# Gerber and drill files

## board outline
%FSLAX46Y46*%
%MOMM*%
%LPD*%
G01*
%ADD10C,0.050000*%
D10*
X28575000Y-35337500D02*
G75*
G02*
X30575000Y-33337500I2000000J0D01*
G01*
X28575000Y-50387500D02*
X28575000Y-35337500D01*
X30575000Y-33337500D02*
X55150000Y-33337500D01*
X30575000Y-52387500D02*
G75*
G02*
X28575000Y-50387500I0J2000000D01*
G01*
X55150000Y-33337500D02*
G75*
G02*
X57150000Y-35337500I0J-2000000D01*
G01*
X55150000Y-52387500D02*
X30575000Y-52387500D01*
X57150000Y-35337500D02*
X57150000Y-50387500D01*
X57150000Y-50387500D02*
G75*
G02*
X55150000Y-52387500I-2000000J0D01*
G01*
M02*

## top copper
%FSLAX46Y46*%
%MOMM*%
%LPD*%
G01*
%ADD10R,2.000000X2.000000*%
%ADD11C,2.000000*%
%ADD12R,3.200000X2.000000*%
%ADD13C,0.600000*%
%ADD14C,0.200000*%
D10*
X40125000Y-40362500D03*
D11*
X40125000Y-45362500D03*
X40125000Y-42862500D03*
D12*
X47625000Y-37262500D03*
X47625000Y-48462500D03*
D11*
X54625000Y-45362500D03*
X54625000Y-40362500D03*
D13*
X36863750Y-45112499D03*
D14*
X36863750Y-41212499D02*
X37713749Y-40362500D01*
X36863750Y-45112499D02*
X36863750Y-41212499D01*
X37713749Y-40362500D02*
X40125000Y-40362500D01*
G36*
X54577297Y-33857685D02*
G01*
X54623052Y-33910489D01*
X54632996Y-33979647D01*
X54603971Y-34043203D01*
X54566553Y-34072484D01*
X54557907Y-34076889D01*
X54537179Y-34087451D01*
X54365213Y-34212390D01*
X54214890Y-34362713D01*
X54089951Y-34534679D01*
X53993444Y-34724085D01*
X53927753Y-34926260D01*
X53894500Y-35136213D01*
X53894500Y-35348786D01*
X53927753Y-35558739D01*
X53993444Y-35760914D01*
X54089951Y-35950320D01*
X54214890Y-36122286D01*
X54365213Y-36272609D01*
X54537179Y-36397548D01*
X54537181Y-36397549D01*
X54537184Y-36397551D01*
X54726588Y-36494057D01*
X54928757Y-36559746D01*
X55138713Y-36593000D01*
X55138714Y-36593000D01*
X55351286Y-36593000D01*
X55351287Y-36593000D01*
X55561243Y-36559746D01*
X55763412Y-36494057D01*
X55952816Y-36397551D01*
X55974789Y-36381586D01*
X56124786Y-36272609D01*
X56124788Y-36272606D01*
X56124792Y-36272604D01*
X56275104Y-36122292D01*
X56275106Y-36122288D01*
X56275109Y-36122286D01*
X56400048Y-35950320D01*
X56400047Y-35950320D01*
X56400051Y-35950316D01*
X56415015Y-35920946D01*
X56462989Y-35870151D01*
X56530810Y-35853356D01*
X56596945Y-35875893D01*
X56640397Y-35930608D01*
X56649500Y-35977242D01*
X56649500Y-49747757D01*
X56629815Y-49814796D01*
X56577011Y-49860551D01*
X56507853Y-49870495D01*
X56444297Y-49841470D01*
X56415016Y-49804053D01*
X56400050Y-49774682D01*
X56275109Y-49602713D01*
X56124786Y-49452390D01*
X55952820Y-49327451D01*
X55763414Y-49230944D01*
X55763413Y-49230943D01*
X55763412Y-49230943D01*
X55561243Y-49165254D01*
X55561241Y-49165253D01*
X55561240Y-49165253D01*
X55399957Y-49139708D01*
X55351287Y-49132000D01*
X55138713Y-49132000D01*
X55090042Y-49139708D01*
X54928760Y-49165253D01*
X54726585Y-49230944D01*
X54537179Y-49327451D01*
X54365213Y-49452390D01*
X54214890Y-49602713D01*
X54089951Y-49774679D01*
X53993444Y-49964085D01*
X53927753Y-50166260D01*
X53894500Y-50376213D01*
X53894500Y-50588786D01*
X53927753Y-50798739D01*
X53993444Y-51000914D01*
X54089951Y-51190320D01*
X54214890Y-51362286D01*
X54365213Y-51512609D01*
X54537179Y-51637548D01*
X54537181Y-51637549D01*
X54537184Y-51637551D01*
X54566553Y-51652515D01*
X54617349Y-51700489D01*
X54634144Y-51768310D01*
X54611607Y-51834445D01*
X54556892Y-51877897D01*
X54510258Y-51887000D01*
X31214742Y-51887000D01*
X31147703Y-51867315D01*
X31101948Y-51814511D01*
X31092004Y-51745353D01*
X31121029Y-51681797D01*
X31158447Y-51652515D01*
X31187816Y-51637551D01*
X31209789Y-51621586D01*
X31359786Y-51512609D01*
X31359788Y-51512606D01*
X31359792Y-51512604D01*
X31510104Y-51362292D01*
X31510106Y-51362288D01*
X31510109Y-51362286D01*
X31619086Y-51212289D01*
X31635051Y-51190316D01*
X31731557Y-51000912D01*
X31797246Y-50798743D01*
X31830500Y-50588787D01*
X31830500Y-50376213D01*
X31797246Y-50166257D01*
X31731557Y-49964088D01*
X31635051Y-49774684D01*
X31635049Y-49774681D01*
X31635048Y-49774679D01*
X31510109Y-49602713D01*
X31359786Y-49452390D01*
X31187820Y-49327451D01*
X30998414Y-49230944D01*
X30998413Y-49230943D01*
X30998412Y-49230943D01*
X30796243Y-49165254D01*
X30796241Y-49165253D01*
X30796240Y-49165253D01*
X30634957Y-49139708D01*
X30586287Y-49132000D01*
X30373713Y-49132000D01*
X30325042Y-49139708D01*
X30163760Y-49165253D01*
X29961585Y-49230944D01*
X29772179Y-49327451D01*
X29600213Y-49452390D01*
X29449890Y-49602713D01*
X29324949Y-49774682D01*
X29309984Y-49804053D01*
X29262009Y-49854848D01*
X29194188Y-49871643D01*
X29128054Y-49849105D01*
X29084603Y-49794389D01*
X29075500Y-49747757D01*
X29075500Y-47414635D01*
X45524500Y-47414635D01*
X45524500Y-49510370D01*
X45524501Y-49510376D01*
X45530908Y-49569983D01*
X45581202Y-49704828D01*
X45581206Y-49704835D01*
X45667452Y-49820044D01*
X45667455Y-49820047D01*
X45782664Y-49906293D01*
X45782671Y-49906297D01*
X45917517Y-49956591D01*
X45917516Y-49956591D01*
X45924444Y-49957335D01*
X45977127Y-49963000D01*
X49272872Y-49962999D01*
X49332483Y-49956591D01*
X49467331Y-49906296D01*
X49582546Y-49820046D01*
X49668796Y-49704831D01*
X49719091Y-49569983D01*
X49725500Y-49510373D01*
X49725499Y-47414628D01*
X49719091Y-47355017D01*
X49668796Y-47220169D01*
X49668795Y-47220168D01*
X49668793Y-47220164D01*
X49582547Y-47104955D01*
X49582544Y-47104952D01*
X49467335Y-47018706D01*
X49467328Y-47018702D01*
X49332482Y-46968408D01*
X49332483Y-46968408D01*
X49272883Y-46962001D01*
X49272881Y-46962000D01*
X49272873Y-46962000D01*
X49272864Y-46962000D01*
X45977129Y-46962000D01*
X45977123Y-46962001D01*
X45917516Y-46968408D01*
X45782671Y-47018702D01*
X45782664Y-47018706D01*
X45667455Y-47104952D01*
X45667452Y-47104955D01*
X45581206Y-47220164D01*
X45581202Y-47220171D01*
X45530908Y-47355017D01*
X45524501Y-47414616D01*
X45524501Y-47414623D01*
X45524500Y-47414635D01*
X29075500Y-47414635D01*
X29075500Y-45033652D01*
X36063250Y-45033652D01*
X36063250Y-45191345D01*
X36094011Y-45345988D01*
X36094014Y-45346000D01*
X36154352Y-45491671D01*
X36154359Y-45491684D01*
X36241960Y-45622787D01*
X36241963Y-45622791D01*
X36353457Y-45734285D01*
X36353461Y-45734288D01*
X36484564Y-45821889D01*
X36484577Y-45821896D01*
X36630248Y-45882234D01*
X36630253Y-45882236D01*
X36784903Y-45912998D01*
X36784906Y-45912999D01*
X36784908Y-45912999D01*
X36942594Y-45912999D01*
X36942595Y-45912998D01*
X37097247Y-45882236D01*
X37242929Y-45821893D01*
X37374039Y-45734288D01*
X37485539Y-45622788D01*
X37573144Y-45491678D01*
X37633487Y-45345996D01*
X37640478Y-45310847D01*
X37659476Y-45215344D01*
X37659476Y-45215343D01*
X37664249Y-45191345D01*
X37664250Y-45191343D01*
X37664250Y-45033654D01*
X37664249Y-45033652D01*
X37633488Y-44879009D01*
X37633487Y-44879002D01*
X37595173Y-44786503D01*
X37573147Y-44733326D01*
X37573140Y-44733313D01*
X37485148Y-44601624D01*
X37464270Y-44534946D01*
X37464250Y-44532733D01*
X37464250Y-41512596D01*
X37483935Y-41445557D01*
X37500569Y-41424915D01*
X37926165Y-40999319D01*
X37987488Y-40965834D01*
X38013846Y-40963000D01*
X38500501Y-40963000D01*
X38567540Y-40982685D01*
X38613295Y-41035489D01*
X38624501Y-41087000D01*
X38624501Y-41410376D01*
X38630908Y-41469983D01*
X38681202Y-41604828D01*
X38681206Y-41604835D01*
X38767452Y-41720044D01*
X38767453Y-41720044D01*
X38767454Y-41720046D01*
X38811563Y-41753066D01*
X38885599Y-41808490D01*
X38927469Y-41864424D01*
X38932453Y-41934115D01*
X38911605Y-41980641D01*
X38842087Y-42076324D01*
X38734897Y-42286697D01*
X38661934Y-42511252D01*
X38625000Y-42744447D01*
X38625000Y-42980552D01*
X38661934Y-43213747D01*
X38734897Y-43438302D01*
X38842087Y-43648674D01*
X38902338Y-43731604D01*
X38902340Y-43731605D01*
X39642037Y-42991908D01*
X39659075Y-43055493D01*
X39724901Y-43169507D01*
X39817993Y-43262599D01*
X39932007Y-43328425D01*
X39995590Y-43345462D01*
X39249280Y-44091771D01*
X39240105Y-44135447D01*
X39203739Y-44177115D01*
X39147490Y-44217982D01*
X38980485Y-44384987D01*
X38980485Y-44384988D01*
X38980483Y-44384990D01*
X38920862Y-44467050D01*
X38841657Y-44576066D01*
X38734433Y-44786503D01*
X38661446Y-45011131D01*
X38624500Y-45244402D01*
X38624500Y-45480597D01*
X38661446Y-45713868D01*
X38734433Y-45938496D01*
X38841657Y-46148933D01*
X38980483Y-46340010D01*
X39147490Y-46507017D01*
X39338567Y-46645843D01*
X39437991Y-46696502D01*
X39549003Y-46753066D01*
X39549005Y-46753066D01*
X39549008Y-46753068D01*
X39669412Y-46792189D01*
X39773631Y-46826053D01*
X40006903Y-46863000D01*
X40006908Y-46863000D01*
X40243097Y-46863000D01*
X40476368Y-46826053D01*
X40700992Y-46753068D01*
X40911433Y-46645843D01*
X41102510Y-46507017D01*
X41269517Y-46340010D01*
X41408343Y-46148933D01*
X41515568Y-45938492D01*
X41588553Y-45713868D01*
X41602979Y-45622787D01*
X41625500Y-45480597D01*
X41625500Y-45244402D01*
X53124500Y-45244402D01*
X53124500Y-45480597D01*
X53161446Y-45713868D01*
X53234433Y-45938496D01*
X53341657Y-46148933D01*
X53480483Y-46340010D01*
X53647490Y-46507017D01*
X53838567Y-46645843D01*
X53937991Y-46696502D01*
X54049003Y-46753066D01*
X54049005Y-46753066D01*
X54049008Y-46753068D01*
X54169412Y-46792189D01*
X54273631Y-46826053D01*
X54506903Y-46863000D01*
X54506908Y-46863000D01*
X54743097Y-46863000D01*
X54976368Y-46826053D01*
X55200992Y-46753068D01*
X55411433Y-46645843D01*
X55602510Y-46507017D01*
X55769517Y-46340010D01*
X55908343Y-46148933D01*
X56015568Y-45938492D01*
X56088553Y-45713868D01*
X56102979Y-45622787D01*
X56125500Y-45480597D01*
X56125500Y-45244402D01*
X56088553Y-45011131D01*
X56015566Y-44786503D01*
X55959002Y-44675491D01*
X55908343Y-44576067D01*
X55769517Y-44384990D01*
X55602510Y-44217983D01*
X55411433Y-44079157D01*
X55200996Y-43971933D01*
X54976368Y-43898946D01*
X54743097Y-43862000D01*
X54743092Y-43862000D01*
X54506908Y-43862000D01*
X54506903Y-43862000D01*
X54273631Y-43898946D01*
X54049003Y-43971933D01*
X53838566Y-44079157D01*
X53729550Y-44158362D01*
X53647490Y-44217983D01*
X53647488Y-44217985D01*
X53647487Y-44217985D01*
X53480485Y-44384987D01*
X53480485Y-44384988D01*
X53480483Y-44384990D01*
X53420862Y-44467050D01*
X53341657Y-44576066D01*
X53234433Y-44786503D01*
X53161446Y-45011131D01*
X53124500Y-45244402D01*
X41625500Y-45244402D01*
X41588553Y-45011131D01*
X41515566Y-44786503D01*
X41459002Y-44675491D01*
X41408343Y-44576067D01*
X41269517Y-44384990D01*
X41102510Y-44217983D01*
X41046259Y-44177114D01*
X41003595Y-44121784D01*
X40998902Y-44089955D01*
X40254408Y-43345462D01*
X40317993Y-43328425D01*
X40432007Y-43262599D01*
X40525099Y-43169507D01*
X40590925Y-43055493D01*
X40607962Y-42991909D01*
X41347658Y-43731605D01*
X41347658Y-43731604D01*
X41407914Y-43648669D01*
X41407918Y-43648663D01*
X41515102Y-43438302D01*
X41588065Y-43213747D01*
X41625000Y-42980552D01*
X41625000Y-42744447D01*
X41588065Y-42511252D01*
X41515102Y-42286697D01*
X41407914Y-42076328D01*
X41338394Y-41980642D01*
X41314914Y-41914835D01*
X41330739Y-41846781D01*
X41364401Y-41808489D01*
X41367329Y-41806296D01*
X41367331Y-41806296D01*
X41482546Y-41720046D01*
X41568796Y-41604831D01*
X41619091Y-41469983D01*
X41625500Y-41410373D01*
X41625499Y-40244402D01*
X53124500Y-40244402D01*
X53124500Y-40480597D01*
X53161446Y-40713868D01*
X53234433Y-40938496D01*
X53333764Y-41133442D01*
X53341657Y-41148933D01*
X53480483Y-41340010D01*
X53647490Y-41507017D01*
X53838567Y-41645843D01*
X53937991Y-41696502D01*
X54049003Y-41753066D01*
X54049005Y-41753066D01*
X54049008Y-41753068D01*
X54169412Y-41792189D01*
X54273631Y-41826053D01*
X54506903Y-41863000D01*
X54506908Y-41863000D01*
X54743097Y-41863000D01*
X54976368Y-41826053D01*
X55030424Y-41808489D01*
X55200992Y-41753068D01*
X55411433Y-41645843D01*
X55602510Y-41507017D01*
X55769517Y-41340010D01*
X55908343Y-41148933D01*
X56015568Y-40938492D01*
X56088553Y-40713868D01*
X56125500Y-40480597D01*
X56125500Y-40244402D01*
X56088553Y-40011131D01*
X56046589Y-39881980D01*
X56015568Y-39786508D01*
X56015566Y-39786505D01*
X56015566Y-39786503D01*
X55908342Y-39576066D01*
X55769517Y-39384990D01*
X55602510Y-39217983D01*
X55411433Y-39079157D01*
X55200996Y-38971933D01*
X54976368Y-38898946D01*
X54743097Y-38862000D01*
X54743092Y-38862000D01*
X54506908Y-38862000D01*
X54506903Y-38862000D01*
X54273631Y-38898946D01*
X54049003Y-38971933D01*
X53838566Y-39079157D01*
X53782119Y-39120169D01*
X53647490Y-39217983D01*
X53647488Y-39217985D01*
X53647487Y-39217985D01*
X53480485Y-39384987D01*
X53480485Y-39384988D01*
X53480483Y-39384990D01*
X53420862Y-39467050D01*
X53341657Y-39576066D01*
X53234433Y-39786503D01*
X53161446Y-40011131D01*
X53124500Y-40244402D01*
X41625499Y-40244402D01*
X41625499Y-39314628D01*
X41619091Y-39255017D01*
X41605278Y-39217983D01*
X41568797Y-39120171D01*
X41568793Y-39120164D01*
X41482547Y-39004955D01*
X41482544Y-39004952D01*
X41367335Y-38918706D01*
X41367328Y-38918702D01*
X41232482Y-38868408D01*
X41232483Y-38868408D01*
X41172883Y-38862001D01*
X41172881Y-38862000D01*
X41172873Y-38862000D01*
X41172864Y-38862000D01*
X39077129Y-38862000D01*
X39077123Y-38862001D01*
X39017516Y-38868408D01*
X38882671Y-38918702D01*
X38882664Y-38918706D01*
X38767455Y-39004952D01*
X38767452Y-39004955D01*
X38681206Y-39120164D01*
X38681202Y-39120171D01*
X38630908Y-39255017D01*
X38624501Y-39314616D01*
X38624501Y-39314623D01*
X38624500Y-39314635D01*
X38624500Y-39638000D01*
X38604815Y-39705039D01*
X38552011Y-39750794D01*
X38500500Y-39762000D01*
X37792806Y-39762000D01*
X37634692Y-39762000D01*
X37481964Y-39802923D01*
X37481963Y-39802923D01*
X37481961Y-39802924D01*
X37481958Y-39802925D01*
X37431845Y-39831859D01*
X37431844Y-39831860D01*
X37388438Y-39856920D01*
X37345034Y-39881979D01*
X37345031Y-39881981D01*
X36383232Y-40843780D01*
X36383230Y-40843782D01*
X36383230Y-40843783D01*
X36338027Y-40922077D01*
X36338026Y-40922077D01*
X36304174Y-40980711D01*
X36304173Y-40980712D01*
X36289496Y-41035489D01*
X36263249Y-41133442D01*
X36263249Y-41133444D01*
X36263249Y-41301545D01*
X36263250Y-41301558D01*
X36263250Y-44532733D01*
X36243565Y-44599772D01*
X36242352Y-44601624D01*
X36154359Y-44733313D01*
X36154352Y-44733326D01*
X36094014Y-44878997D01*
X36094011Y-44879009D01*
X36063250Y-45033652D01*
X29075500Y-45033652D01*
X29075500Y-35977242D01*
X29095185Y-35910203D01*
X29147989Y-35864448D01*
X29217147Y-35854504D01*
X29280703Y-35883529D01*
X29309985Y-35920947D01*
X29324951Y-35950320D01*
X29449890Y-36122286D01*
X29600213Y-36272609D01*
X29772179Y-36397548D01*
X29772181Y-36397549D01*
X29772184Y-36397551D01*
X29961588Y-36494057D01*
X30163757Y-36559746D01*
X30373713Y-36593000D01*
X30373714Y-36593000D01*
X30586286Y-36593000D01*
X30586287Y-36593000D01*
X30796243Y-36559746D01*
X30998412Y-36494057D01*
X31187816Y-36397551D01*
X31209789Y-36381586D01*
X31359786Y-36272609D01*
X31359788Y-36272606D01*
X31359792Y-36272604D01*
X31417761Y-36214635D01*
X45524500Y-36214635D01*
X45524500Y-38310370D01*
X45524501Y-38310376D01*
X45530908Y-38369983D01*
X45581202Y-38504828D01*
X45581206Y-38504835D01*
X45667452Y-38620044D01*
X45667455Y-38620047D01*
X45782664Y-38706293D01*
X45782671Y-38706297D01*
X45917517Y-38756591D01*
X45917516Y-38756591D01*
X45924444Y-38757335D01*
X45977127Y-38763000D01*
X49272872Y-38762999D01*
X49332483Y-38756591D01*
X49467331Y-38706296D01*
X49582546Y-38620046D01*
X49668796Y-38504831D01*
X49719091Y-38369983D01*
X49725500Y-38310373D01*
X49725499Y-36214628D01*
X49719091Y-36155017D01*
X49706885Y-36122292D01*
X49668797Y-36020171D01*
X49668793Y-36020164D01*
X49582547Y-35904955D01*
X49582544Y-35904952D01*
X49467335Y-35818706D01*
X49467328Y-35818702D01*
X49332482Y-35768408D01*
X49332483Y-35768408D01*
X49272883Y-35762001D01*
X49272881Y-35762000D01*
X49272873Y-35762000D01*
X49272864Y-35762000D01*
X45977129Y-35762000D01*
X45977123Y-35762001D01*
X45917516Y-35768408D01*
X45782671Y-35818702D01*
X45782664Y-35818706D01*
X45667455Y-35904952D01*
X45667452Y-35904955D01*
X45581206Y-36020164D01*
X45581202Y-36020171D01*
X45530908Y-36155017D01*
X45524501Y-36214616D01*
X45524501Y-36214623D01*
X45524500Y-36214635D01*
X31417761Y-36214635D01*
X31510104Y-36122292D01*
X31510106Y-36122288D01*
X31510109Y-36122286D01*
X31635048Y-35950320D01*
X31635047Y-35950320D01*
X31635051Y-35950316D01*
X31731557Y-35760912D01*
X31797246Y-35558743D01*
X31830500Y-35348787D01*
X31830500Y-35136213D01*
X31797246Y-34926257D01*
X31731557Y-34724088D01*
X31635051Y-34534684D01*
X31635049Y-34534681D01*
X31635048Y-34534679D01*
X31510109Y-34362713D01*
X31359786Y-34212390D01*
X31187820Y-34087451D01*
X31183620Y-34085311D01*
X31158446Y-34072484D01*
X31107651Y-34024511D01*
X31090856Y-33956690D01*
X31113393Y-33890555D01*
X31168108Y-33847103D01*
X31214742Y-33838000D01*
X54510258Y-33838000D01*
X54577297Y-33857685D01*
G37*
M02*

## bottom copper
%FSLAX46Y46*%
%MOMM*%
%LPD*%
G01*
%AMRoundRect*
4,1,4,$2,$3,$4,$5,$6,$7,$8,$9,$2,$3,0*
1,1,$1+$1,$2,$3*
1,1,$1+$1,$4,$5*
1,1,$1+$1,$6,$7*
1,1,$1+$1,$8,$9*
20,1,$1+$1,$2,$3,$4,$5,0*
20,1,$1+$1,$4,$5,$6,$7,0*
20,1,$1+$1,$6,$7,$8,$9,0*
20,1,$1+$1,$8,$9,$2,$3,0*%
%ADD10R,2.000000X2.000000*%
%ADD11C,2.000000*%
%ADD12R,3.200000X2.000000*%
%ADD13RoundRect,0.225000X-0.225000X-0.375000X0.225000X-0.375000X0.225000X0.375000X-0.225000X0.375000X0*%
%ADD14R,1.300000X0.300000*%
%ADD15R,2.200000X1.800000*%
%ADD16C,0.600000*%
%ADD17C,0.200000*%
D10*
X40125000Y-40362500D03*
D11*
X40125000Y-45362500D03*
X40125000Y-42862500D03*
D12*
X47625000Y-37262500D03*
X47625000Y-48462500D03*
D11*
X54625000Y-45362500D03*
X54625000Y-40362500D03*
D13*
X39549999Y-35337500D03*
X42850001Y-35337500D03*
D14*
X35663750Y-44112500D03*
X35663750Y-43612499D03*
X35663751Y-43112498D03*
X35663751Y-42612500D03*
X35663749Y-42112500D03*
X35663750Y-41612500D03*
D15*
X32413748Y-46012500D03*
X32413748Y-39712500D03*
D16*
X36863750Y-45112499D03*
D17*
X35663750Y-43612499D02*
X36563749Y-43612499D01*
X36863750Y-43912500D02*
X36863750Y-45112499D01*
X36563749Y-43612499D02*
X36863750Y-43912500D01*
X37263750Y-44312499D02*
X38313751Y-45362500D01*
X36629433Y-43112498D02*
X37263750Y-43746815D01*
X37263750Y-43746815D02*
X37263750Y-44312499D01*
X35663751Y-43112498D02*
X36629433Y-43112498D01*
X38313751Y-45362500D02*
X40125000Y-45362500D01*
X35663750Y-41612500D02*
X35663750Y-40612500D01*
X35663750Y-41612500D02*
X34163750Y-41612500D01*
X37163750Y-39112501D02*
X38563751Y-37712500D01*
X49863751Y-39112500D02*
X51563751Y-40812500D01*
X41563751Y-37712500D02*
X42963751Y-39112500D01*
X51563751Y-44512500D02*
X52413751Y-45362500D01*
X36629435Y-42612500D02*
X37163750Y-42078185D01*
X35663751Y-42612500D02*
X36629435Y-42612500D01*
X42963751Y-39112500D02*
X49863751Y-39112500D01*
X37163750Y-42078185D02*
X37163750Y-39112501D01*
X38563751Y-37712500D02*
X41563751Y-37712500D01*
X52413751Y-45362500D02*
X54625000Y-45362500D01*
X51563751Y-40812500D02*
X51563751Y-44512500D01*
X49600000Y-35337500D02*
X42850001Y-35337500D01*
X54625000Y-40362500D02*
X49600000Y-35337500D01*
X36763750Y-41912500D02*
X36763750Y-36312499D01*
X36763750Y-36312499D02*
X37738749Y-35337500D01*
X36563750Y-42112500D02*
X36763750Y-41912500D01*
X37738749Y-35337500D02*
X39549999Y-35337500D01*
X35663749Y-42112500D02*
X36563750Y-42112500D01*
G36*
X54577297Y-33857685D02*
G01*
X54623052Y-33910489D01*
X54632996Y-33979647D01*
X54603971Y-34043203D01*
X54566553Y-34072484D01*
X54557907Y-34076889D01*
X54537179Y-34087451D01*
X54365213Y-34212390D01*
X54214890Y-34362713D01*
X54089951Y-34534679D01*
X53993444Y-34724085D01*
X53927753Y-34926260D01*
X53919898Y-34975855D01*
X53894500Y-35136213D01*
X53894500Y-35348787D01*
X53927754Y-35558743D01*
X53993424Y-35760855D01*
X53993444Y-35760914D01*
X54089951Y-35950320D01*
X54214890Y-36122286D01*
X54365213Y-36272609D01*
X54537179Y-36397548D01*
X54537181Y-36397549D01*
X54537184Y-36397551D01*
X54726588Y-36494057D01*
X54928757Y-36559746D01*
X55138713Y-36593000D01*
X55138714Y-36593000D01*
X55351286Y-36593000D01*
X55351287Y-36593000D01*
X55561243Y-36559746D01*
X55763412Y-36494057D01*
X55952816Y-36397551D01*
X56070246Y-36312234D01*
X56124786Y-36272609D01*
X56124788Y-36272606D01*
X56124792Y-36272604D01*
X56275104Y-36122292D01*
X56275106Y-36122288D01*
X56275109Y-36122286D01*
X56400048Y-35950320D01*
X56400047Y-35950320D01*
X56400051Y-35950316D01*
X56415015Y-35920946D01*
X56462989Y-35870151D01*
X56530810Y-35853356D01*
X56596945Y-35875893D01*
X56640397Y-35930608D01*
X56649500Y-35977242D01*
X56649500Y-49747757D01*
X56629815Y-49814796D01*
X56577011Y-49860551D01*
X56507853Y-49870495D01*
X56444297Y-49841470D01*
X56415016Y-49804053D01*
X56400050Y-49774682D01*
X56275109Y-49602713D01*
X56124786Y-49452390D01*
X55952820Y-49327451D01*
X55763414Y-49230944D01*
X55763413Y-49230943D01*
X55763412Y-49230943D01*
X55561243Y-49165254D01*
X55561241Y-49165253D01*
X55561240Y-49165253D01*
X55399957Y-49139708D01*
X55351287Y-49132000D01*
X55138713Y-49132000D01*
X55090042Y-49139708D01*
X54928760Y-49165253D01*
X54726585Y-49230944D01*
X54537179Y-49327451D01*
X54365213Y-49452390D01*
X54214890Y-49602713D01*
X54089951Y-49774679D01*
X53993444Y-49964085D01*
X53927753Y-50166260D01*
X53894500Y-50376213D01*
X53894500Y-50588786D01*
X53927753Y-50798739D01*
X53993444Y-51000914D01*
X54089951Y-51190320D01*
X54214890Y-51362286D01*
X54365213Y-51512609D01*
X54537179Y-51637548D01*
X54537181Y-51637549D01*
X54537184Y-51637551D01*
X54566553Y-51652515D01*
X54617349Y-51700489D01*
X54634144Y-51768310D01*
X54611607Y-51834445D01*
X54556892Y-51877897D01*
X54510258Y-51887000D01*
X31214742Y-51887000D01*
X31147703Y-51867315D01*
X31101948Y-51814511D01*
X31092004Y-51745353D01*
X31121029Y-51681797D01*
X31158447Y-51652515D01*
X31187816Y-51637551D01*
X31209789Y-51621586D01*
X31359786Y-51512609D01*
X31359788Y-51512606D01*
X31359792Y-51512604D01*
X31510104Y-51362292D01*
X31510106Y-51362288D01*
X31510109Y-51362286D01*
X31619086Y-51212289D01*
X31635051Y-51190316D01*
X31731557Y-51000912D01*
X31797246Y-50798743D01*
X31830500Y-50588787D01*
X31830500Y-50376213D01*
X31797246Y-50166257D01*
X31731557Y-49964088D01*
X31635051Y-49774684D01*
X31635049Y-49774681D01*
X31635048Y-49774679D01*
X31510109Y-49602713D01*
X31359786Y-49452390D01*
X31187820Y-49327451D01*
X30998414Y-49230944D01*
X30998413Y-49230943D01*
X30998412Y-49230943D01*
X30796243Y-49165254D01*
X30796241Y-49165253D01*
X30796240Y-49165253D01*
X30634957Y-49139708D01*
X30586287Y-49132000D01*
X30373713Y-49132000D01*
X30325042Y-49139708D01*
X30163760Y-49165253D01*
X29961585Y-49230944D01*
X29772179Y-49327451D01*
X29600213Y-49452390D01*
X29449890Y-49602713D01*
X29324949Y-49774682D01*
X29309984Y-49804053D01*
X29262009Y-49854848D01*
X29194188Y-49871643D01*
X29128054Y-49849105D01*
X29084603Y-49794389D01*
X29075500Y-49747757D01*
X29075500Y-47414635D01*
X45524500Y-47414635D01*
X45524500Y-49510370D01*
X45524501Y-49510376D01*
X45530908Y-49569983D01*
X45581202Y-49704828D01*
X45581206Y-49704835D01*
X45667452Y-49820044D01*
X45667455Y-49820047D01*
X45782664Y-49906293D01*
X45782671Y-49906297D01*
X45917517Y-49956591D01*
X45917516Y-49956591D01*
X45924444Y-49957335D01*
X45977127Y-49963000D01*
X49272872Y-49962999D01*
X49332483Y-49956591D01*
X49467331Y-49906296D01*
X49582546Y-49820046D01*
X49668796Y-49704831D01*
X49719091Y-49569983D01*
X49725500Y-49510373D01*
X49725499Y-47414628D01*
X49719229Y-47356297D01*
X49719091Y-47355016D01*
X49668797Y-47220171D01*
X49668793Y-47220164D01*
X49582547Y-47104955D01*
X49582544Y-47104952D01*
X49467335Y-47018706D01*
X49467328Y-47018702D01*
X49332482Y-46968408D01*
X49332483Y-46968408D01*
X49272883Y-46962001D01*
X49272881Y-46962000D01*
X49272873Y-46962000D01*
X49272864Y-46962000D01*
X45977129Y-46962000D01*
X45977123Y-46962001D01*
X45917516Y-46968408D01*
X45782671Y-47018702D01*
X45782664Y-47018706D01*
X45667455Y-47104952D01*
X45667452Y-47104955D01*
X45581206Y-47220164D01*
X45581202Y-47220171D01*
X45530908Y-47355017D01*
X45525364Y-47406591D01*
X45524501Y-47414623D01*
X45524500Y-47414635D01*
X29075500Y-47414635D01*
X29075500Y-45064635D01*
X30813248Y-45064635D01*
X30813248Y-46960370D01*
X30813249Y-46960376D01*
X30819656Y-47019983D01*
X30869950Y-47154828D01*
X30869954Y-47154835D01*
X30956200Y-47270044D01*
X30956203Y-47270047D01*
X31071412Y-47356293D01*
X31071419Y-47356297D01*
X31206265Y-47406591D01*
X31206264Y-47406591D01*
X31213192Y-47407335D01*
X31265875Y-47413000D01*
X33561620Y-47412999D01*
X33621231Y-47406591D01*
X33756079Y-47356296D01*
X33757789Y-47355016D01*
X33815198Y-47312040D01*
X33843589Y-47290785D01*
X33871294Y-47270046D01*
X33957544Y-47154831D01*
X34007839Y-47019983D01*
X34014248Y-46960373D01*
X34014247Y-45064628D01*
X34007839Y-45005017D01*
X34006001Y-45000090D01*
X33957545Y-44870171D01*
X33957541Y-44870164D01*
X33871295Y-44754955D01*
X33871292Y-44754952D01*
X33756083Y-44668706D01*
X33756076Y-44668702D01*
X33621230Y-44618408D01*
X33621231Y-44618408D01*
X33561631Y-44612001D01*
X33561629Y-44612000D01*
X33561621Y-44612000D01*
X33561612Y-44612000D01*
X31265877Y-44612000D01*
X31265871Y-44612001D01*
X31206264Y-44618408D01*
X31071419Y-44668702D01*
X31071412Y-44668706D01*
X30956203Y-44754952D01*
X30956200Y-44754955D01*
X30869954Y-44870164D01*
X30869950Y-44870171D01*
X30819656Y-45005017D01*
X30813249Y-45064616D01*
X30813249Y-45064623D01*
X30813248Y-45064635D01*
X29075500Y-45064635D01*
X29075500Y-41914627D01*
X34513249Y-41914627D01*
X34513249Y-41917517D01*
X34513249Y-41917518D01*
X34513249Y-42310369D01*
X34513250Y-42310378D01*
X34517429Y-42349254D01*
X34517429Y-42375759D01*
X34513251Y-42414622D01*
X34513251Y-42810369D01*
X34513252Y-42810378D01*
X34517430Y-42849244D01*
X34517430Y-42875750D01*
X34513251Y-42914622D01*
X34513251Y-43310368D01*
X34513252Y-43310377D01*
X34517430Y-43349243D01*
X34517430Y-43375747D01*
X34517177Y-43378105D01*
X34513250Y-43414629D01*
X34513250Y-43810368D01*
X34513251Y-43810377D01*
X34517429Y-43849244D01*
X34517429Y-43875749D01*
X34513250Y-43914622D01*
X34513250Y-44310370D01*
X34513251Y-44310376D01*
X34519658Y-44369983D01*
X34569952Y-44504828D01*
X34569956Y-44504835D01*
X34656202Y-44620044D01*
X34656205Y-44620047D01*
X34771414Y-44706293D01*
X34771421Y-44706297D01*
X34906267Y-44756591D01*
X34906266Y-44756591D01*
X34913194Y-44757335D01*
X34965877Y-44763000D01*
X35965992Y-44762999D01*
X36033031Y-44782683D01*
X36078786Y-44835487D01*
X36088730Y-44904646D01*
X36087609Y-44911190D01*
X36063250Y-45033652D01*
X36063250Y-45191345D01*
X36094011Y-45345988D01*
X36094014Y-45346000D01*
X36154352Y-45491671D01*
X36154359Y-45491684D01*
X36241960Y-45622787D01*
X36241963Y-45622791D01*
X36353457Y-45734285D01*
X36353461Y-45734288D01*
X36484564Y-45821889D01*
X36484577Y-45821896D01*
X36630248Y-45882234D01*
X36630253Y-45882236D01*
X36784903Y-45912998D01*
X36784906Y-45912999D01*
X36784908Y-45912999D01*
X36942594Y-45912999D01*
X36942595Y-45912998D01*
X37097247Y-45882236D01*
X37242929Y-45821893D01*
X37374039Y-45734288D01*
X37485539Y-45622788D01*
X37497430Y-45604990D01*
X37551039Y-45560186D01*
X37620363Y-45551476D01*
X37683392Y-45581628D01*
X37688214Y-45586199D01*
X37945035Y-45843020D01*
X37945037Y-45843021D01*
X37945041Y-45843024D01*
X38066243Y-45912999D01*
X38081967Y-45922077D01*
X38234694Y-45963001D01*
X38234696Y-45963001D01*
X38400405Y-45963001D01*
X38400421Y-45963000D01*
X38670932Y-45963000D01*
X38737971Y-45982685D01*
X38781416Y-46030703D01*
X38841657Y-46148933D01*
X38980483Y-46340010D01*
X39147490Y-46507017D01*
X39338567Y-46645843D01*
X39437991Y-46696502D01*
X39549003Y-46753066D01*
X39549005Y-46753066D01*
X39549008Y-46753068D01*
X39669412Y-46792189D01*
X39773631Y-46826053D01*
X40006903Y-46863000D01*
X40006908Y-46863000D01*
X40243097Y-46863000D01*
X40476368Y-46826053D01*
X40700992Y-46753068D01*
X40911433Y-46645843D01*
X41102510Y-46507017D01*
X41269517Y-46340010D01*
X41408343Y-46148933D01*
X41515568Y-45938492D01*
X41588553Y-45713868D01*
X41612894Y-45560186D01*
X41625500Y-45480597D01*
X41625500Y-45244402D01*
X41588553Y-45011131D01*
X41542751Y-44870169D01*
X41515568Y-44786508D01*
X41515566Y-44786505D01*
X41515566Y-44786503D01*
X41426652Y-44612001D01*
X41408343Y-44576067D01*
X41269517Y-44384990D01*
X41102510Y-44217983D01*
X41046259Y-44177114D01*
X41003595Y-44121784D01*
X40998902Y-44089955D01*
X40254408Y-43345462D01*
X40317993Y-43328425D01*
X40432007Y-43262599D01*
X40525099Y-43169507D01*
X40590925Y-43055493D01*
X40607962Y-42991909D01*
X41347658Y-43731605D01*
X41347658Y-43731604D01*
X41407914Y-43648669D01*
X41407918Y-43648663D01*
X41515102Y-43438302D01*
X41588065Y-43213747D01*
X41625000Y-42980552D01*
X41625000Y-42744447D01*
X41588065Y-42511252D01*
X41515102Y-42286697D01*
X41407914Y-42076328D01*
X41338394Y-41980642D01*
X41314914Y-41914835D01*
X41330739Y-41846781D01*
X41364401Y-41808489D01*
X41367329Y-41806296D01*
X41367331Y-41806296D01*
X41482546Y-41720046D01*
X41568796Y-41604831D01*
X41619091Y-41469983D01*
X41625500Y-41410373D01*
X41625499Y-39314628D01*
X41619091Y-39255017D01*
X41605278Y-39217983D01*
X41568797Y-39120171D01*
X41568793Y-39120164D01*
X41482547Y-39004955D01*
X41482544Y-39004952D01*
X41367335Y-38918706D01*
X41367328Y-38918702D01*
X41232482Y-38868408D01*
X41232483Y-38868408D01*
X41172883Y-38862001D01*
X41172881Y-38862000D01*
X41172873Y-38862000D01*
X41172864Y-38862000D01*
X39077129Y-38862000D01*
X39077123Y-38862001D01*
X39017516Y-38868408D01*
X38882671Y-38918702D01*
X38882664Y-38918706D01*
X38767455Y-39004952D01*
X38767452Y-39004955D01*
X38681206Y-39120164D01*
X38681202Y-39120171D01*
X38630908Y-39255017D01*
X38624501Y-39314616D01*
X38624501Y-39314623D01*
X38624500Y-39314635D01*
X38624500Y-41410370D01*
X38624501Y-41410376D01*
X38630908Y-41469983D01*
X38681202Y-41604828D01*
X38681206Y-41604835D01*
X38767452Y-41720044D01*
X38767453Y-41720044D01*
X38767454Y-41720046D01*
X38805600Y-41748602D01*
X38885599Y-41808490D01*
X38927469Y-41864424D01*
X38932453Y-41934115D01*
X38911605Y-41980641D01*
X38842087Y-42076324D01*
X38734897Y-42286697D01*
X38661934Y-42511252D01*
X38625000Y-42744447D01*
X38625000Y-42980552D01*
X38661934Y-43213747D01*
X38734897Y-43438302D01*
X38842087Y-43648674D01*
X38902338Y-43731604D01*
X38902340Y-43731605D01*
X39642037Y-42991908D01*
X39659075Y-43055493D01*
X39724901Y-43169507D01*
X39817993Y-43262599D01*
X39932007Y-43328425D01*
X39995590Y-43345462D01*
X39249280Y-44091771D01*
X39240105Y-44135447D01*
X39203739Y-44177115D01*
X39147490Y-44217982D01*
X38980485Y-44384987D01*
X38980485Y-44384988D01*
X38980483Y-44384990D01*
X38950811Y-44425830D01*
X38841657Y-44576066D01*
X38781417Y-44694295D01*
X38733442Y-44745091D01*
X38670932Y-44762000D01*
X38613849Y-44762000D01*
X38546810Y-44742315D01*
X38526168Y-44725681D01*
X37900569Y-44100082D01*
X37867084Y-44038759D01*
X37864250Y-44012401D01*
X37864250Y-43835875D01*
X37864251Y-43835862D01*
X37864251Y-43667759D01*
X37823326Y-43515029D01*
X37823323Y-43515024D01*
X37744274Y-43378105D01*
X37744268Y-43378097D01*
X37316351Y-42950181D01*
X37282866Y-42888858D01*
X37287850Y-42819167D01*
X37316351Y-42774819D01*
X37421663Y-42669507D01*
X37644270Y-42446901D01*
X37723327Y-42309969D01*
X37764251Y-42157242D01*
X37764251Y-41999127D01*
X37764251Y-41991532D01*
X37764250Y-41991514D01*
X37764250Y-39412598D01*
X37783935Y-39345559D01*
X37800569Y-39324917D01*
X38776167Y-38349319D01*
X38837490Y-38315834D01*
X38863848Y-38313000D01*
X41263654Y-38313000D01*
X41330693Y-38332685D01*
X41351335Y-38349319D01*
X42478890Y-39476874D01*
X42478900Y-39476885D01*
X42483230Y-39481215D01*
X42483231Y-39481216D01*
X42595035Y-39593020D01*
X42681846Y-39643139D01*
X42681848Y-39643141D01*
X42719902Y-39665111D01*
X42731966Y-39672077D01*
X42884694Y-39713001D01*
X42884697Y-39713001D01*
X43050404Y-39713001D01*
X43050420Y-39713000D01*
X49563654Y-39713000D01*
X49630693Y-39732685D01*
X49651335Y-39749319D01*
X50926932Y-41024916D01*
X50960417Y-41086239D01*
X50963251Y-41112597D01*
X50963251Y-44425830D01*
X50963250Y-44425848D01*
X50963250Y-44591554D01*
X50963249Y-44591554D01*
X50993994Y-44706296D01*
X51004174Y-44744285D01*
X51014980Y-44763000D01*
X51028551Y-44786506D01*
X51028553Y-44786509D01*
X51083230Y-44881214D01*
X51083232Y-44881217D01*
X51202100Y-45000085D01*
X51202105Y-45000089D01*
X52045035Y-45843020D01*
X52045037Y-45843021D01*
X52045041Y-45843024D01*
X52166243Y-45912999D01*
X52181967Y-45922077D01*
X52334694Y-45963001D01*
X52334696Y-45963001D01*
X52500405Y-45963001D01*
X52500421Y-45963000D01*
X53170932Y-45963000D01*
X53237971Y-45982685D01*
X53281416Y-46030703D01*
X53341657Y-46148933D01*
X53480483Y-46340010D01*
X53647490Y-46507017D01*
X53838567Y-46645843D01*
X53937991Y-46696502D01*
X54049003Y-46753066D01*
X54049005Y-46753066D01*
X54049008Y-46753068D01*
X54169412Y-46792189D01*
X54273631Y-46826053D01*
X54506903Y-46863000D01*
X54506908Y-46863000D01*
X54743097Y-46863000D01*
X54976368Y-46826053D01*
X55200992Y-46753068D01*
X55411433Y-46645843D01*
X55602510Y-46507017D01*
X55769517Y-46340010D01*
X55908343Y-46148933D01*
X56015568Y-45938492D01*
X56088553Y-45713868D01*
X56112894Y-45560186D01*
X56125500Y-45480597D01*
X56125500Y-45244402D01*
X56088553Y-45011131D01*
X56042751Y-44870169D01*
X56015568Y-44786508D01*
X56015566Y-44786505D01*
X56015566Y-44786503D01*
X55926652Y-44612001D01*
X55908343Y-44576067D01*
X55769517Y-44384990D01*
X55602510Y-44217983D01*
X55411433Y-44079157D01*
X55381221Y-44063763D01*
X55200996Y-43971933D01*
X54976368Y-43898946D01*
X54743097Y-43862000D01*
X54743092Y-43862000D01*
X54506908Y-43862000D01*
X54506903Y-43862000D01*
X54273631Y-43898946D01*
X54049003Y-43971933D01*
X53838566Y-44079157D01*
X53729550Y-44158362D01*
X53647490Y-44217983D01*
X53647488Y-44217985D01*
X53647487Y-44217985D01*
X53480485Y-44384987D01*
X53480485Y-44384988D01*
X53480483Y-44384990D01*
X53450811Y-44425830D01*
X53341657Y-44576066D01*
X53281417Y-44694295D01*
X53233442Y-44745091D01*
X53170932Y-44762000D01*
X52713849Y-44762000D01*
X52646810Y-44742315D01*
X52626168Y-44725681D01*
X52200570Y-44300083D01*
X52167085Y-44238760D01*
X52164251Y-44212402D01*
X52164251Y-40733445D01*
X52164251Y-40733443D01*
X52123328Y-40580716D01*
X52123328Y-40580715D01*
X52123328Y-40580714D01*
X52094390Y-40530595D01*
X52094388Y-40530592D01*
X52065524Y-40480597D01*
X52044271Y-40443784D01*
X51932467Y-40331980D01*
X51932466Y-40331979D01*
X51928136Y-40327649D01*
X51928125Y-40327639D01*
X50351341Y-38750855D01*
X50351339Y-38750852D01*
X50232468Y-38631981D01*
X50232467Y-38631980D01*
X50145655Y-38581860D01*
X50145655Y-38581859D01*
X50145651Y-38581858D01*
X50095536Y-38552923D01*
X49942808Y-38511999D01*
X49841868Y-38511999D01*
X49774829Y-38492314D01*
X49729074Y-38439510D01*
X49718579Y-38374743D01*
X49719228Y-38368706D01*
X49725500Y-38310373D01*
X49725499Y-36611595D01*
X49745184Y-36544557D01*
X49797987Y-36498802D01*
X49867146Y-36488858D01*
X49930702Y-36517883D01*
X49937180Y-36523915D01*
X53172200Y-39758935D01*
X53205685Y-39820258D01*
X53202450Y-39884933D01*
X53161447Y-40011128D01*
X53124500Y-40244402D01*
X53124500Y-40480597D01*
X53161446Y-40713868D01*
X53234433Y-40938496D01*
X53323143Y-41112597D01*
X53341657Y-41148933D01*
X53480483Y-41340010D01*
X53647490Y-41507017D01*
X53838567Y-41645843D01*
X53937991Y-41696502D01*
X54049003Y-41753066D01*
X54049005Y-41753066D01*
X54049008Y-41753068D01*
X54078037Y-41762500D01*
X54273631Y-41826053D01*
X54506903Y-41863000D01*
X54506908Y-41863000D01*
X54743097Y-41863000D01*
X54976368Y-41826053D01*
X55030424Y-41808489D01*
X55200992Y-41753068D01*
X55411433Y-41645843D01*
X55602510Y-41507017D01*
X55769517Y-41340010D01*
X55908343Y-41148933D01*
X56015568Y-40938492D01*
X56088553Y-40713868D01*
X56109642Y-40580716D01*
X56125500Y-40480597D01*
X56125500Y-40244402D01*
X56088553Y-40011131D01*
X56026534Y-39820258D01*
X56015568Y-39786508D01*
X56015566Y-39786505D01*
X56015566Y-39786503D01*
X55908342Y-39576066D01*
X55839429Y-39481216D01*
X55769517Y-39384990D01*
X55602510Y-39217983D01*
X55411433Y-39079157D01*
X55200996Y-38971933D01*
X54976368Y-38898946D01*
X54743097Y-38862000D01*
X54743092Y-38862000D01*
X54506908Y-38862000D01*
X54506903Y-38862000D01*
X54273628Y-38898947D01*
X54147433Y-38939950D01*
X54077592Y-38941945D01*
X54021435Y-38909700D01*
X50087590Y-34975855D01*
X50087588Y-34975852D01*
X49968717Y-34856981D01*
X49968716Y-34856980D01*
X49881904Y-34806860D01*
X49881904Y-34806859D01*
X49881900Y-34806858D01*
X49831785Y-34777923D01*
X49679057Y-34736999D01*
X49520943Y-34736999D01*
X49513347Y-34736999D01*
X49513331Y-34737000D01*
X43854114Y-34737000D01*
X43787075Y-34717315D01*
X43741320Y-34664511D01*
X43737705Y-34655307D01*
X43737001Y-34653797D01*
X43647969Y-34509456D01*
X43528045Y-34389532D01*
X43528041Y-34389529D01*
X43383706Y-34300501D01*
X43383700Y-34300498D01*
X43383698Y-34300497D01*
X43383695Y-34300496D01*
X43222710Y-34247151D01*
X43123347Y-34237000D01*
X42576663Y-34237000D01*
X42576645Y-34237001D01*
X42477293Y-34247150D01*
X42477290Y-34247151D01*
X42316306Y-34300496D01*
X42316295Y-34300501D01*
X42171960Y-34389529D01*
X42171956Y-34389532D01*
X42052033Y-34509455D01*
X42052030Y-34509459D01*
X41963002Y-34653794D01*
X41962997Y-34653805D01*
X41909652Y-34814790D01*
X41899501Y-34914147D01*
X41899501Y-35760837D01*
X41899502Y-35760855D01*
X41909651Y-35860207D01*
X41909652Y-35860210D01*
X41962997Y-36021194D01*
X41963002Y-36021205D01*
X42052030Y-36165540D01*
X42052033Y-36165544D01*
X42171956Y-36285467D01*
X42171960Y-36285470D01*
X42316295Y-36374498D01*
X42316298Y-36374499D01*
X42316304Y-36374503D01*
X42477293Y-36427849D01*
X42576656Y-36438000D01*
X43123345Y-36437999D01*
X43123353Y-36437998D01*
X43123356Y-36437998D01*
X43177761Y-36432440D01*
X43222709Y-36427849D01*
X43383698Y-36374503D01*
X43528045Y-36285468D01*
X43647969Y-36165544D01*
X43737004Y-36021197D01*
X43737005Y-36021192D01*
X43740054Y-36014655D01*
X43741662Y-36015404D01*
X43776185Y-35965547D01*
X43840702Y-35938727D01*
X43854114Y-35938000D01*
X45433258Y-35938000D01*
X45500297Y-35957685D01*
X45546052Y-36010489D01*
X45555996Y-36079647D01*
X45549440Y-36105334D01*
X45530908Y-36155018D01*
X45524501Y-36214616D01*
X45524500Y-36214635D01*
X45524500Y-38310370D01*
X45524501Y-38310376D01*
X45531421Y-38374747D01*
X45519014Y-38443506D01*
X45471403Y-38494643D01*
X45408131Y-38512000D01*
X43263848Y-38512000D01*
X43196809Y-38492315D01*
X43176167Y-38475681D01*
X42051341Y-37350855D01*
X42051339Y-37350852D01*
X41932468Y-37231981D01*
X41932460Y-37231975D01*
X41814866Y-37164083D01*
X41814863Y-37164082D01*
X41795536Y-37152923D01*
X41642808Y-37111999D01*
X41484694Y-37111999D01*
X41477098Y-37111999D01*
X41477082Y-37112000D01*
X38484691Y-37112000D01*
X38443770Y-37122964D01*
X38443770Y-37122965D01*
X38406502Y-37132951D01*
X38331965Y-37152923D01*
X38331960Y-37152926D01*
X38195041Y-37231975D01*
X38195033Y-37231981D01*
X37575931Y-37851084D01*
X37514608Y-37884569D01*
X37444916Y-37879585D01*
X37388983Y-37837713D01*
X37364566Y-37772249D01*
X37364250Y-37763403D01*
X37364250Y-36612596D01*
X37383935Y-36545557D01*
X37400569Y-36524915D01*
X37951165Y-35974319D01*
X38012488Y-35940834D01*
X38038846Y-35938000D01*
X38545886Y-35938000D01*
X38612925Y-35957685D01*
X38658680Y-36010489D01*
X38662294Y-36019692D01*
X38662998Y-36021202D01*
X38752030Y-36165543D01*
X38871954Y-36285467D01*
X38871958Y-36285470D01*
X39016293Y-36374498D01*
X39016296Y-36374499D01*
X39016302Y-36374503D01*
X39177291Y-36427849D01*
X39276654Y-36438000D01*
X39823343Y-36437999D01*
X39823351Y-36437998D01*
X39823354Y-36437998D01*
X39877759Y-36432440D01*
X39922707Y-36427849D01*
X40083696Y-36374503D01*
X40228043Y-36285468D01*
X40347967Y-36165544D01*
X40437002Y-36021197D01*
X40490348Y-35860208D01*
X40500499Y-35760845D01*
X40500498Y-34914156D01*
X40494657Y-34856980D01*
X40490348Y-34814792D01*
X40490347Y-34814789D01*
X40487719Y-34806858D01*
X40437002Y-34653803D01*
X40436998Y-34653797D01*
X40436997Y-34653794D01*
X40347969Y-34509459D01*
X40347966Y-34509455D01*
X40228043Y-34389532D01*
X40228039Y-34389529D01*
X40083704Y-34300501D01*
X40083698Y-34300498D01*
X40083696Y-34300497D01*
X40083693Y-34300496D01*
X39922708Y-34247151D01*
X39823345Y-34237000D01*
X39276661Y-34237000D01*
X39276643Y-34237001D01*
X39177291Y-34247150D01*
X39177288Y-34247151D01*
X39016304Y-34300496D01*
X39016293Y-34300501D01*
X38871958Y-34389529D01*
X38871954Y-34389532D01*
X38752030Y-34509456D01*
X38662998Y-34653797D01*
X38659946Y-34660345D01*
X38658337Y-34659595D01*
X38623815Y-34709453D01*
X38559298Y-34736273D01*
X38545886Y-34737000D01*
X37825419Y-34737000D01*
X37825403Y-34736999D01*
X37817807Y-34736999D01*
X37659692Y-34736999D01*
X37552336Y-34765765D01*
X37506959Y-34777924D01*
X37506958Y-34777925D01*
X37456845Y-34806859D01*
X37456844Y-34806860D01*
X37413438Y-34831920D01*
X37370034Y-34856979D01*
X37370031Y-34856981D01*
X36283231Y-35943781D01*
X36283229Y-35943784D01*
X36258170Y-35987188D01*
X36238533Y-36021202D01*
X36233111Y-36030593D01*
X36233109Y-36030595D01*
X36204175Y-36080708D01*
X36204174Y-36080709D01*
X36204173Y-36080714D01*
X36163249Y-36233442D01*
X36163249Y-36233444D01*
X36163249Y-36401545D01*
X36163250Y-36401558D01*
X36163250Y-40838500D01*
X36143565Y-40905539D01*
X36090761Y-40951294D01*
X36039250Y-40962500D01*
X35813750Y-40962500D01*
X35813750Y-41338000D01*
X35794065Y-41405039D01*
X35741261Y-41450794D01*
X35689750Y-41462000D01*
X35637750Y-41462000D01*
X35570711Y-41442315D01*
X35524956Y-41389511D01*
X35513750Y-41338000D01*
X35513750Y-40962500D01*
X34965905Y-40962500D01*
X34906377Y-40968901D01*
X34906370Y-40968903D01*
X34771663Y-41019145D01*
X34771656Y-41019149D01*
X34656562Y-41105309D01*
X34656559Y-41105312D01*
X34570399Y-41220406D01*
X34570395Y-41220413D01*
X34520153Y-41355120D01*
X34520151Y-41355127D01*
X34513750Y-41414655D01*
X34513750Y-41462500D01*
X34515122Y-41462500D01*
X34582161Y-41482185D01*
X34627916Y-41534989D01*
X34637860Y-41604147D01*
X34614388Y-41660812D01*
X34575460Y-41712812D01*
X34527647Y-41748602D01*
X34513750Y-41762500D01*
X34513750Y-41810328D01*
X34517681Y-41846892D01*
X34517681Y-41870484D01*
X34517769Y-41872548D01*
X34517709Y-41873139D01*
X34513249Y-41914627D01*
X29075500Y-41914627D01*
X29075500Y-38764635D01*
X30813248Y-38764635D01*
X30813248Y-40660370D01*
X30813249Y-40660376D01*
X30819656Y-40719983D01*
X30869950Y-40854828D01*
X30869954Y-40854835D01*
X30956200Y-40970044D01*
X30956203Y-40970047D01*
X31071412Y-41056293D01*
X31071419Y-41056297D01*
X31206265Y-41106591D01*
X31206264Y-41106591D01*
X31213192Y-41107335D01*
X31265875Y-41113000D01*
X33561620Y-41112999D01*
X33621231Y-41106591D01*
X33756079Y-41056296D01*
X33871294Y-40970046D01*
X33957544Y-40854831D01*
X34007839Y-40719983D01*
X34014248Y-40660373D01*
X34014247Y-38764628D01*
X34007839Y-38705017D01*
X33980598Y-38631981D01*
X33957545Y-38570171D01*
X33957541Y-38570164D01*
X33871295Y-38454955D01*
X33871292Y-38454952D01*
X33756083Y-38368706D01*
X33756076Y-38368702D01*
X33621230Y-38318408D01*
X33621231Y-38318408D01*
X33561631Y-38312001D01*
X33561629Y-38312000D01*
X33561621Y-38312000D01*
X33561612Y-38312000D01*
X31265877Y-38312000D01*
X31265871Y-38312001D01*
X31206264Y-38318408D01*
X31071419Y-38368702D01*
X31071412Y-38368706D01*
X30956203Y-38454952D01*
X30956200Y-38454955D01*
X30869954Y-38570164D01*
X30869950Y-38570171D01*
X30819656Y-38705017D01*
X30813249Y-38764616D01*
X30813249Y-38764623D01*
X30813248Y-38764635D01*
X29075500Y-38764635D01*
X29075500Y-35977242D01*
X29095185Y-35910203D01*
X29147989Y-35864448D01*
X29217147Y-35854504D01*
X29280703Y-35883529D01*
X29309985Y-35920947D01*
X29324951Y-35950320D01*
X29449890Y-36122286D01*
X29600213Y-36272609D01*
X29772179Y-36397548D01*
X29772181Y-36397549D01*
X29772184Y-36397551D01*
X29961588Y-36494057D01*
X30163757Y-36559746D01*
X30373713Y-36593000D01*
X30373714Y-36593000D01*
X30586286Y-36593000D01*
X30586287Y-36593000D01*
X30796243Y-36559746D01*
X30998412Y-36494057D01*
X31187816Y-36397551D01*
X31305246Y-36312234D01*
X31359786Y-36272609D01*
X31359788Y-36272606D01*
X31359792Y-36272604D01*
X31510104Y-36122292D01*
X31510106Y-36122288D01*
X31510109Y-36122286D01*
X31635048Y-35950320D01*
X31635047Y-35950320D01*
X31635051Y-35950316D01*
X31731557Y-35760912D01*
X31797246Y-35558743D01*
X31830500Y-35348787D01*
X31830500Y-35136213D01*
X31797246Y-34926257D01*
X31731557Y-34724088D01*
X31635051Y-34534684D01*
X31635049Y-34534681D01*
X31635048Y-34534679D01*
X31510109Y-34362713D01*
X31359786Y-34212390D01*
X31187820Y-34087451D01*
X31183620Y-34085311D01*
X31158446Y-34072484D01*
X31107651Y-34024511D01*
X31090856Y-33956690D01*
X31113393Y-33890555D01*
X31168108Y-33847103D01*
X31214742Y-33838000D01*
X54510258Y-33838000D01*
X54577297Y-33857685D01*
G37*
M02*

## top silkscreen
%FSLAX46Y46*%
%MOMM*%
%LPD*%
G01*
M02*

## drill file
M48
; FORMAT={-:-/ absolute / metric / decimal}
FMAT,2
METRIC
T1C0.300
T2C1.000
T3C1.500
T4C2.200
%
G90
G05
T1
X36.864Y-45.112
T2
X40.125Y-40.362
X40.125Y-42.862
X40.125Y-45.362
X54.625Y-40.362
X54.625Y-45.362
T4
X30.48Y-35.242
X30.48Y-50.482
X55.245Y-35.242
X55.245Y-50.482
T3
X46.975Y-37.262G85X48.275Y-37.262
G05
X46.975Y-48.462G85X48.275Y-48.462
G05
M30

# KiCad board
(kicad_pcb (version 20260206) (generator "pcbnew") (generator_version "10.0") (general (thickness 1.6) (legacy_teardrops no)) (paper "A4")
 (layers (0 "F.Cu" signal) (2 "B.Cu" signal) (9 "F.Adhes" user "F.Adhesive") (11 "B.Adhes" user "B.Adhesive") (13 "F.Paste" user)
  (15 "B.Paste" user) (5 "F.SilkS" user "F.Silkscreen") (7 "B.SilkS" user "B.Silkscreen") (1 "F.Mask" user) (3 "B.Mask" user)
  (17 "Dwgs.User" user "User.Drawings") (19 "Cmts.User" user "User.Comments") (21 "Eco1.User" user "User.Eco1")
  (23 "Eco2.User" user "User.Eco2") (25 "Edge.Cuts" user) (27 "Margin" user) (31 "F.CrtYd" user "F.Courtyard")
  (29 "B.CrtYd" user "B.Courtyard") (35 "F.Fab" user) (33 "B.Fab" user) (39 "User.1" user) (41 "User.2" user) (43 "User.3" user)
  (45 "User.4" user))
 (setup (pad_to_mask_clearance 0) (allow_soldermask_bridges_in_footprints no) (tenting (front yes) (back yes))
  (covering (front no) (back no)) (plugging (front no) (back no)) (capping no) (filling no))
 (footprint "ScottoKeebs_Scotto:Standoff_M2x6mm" (layer "F.Cu") (at 30.48 50.4825)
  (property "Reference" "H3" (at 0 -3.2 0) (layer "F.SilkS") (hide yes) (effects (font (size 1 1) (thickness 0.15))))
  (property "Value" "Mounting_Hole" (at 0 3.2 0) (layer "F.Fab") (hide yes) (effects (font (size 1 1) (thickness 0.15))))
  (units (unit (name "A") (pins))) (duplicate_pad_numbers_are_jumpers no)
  (pad "" np_thru_hole circle (at 0 0) (size 2.2 2.2) (drill 2.2) (layers "*.Cu" "*.Mask")))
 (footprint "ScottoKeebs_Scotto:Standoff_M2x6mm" (layer "F.Cu") (at 55.245 35.2425)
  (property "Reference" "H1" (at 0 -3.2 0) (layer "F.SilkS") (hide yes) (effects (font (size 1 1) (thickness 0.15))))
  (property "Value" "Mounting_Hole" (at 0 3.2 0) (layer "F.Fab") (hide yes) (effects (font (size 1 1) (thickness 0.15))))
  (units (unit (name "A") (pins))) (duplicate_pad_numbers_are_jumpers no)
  (pad "" np_thru_hole circle (at 0 0) (size 2.2 2.2) (drill 2.2) (layers "*.Cu" "*.Mask")))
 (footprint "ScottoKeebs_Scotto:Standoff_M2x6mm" (layer "F.Cu") (at 30.48 35.2425)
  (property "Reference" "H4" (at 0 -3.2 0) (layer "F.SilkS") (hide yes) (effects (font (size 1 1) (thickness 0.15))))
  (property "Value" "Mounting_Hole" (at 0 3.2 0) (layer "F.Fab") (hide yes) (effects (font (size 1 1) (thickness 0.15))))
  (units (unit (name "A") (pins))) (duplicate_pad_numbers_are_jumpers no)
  (pad "" np_thru_hole circle (at 0 0) (size 2.2 2.2) (drill 2.2) (layers "*.Cu" "*.Mask")))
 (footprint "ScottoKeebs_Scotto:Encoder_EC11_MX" (layer "F.Cu") (at 47.625 42.8625)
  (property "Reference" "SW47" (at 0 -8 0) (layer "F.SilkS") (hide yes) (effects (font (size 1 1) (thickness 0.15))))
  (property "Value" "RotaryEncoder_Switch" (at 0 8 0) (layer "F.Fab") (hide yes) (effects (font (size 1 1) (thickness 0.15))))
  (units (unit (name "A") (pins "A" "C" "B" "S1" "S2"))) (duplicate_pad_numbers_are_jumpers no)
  (pad "A" thru_hole rect (at -7.5 -2.5) (size 2 2) (drill 1) (layers "*.Cu" "*.Mask") (remove_unused_layers no) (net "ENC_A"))
  (pad "B" thru_hole circle (at -7.5 2.5) (size 2 2) (drill 1) (layers "*.Cu" "*.Mask") (remove_unused_layers no) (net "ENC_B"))
  (pad "C" thru_hole circle (at -7.5 0) (size 2 2) (drill 1) (layers "*.Cu" "*.Mask") (remove_unused_layers no) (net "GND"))
  (pad "MP" thru_hole rect (at 0 -5.6) (size 3.2 2) (drill oval 2.8 1.5) (layers "*.Cu" "*.Mask") (remove_unused_layers no))
  (pad "MP" thru_hole rect (at 0 5.6) (size 3.2 2) (drill oval 2.8 1.5) (layers "*.Cu" "*.Mask") (remove_unused_layers no))
  (pad "S1" thru_hole circle (at 7 2.5) (size 2 2) (drill 1) (layers "*.Cu" "*.Mask") (remove_unused_layers no) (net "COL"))
  (pad "S2" thru_hole circle (at 7 -2.5) (size 2 2) (drill 1) (layers "*.Cu" "*.Mask") (remove_unused_layers no) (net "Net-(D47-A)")))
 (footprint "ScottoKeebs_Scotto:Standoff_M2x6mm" (layer "F.Cu") (at 55.245 50.4825)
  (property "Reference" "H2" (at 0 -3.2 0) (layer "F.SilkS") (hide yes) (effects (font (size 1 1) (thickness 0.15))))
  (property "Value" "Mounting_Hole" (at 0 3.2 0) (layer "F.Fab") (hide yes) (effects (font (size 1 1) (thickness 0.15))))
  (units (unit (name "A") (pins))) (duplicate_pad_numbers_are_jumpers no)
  (pad "" np_thru_hole circle (at 0 0) (size 2.2 2.2) (drill 2.2) (layers "*.Cu" "*.Mask")))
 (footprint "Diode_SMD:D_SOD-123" (layer "B.Cu") (at 41.2 35.3375)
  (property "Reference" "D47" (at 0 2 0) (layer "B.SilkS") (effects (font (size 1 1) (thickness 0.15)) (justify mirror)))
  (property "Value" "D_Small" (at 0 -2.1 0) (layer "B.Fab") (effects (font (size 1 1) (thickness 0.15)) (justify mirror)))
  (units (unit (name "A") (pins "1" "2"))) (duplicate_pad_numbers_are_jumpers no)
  (pad "1" smd roundrect (at -1.650001 0) (size 0.9 1.2) (layers "B.Cu" "B.Mask" "B.Paste") (roundrect_rratio 0.25) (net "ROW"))
  (pad "2" smd roundrect (at 1.650001 0) (size 0.9 1.2) (layers "B.Cu" "B.Mask" "B.Paste") (roundrect_rratio 0.25) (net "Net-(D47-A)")))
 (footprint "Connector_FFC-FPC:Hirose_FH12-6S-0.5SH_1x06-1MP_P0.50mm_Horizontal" (layer "B.Cu") (at 33.81375 42.8625 90)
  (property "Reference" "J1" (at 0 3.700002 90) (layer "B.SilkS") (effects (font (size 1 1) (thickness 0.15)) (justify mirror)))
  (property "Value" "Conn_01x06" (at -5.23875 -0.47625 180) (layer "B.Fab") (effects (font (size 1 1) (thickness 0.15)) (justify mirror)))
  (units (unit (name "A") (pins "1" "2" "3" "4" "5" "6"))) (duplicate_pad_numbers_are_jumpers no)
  (pad "1" smd rect (at -1.25 1.85 90) (size 0.3 1.3) (layers "B.Cu" "B.Mask" "B.Paste") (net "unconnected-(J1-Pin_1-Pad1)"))
  (pad "2" smd rect (at -0.749999 1.85 90) (size 0.3 1.3) (layers "B.Cu" "B.Mask" "B.Paste") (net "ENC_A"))
  (pad "3" smd rect (at -0.249998 1.850001 90) (size 0.3 1.3) (layers "B.Cu" "B.Mask" "B.Paste") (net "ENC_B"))
  (pad "4" smd rect (at 0.25 1.850001 90) (size 0.3 1.3) (layers "B.Cu" "B.Mask" "B.Paste") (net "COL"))
  (pad "5" smd rect (at 0.75 1.849999 90) (size 0.3 1.3) (layers "B.Cu" "B.Mask" "B.Paste") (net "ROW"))
  (pad "6" smd rect (at 1.25 1.85 90) (size 0.3 1.3) (layers "B.Cu" "B.Mask" "B.Paste") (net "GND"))
  (pad "MP" smd rect (at -3.15 -1.400002 90) (size 1.8 2.2) (layers "B.Cu" "B.Mask" "B.Paste"))
  (pad "MP" smd rect (at 3.15 -1.400002 90) (size 1.8 2.2) (layers "B.Cu" "B.Mask" "B.Paste")))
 (gr_arc (start 28.575 35.3375) (mid 29.160786 33.923286) (end 30.575 33.3375) (stroke (width 0.05) (type default)) (layer "Edge.Cuts"))
 (gr_line (start 28.575 50.3875) (end 28.575 35.3375) (stroke (width 0.05) (type default)) (layer "Edge.Cuts"))
 (gr_line (start 30.575 33.3375) (end 55.15 33.3375) (stroke (width 0.05) (type default)) (layer "Edge.Cuts"))
 (gr_arc (start 30.575 52.3875) (mid 29.160786 51.801714) (end 28.575 50.3875) (stroke (width 0.05) (type default)) (layer "Edge.Cuts"))
 (gr_arc (start 55.15 33.3375) (mid 56.564214 33.923286) (end 57.15 35.3375) (stroke (width 0.05) (type default)) (layer "Edge.Cuts"))
 (gr_line (start 55.15 52.3875) (end 30.575 52.3875) (stroke (width 0.05) (type default)) (layer "Edge.Cuts"))
 (gr_line (start 57.15 35.3375) (end 57.15 50.3875) (stroke (width 0.05) (type default)) (layer "Edge.Cuts"))
 (gr_arc (start 57.15 50.3875) (mid 56.564214 51.801714) (end 55.15 52.3875) (stroke (width 0.05) (type default)) (layer "Edge.Cuts"))
 (segment (start 36.86375 41.212499) (end 37.713749 40.3625) (width 0.2) (layer "F.Cu") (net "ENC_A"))
 (segment (start 36.86375 45.112499) (end 36.86375 41.212499) (width 0.2) (layer "F.Cu") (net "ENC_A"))
 (segment (start 37.713749 40.3625) (end 40.125 40.3625) (width 0.2) (layer "F.Cu") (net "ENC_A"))
 (via (at 36.86375 45.112499) (size 0.6) (drill 0.3) (layers "F.Cu" "B.Cu") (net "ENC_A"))
 (segment (start 35.66375 43.612499) (end 36.563749 43.612499) (width 0.2) (layer "B.Cu") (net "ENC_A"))
 (segment (start 36.86375 43.9125) (end 36.86375 45.112499) (width 0.2) (layer "B.Cu") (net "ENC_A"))
 (segment (start 36.563749 43.612499) (end 36.86375 43.9125) (width 0.2) (layer "B.Cu") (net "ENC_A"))
 (segment (start 37.26375 44.312499) (end 38.313751 45.3625) (width 0.2) (layer "B.Cu") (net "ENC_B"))
 (segment (start 36.629433 43.112498) (end 37.26375 43.746815) (width 0.2) (layer "B.Cu") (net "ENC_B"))
 (segment (start 37.26375 43.746815) (end 37.26375 44.312499) (width 0.2) (layer "B.Cu") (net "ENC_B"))
 (segment (start 35.663751 43.112498) (end 36.629433 43.112498) (width 0.2) (layer "B.Cu") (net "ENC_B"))
 (segment (start 38.313751 45.3625) (end 40.125 45.3625) (width 0.2) (layer "B.Cu") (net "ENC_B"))
 (segment (start 35.66375 41.6125) (end 35.66375 40.6125) (width 0.2) (layer "B.Cu") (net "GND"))
 (segment (start 35.66375 41.6125) (end 34.16375 41.6125) (width 0.2) (layer "B.Cu") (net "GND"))
 (segment (start 37.16375 39.112501) (end 38.563751 37.7125) (width 0.2) (layer "B.Cu") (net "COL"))
 (segment (start 49.863751 39.1125) (end 51.563751 40.8125) (width 0.2) (layer "B.Cu") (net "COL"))
 (segment (start 41.563751 37.7125) (end 42.963751 39.1125) (width 0.2) (layer "B.Cu") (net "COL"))
 (segment (start 51.563751 44.5125) (end 52.413751 45.3625) (width 0.2) (layer "B.Cu") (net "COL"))
 (segment (start 36.629435 42.6125) (end 37.16375 42.078185) (width 0.2) (layer "B.Cu") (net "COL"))
 (segment (start 35.663751 42.6125) (end 36.629435 42.6125) (width 0.2) (layer "B.Cu") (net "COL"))
 (segment (start 42.963751 39.1125) (end 49.863751 39.1125) (width 0.2) (layer "B.Cu") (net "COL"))
 (segment (start 37.16375 42.078185) (end 37.16375 39.112501) (width 0.2) (layer "B.Cu") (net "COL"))
 (segment (start 38.563751 37.7125) (end 41.563751 37.7125) (width 0.2) (layer "B.Cu") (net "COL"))
 (segment (start 52.413751 45.3625) (end 54.625 45.3625) (width 0.2) (layer "B.Cu") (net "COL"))
 (segment (start 51.563751 40.8125) (end 51.563751 44.5125) (width 0.2) (layer "B.Cu") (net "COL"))
 (segment (start 49.6 35.3375) (end 42.850001 35.3375) (width 0.2) (layer "B.Cu") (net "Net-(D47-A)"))
 (segment (start 54.625 40.3625) (end 49.6 35.3375) (width 0.2) (layer "B.Cu") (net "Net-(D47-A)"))
 (segment (start 36.76375 41.9125) (end 36.76375 36.312499) (width 0.2) (layer "B.Cu") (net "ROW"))
 (segment (start 36.76375 36.312499) (end 37.738749 35.3375) (width 0.2) (layer "B.Cu") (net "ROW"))
 (segment (start 36.56375 42.1125) (end 36.76375 41.9125) (width 0.2) (layer "B.Cu") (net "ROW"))
 (segment (start 37.738749 35.3375) (end 39.549999 35.3375) (width 0.2) (layer "B.Cu") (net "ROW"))
 (segment (start 35.663749 42.1125) (end 36.56375 42.1125) (width 0.2) (layer "B.Cu") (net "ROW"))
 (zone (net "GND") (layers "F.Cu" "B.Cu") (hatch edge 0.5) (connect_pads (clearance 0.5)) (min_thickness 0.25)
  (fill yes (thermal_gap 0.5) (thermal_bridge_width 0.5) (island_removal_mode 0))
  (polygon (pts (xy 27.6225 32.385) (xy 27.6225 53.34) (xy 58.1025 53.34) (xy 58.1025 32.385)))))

